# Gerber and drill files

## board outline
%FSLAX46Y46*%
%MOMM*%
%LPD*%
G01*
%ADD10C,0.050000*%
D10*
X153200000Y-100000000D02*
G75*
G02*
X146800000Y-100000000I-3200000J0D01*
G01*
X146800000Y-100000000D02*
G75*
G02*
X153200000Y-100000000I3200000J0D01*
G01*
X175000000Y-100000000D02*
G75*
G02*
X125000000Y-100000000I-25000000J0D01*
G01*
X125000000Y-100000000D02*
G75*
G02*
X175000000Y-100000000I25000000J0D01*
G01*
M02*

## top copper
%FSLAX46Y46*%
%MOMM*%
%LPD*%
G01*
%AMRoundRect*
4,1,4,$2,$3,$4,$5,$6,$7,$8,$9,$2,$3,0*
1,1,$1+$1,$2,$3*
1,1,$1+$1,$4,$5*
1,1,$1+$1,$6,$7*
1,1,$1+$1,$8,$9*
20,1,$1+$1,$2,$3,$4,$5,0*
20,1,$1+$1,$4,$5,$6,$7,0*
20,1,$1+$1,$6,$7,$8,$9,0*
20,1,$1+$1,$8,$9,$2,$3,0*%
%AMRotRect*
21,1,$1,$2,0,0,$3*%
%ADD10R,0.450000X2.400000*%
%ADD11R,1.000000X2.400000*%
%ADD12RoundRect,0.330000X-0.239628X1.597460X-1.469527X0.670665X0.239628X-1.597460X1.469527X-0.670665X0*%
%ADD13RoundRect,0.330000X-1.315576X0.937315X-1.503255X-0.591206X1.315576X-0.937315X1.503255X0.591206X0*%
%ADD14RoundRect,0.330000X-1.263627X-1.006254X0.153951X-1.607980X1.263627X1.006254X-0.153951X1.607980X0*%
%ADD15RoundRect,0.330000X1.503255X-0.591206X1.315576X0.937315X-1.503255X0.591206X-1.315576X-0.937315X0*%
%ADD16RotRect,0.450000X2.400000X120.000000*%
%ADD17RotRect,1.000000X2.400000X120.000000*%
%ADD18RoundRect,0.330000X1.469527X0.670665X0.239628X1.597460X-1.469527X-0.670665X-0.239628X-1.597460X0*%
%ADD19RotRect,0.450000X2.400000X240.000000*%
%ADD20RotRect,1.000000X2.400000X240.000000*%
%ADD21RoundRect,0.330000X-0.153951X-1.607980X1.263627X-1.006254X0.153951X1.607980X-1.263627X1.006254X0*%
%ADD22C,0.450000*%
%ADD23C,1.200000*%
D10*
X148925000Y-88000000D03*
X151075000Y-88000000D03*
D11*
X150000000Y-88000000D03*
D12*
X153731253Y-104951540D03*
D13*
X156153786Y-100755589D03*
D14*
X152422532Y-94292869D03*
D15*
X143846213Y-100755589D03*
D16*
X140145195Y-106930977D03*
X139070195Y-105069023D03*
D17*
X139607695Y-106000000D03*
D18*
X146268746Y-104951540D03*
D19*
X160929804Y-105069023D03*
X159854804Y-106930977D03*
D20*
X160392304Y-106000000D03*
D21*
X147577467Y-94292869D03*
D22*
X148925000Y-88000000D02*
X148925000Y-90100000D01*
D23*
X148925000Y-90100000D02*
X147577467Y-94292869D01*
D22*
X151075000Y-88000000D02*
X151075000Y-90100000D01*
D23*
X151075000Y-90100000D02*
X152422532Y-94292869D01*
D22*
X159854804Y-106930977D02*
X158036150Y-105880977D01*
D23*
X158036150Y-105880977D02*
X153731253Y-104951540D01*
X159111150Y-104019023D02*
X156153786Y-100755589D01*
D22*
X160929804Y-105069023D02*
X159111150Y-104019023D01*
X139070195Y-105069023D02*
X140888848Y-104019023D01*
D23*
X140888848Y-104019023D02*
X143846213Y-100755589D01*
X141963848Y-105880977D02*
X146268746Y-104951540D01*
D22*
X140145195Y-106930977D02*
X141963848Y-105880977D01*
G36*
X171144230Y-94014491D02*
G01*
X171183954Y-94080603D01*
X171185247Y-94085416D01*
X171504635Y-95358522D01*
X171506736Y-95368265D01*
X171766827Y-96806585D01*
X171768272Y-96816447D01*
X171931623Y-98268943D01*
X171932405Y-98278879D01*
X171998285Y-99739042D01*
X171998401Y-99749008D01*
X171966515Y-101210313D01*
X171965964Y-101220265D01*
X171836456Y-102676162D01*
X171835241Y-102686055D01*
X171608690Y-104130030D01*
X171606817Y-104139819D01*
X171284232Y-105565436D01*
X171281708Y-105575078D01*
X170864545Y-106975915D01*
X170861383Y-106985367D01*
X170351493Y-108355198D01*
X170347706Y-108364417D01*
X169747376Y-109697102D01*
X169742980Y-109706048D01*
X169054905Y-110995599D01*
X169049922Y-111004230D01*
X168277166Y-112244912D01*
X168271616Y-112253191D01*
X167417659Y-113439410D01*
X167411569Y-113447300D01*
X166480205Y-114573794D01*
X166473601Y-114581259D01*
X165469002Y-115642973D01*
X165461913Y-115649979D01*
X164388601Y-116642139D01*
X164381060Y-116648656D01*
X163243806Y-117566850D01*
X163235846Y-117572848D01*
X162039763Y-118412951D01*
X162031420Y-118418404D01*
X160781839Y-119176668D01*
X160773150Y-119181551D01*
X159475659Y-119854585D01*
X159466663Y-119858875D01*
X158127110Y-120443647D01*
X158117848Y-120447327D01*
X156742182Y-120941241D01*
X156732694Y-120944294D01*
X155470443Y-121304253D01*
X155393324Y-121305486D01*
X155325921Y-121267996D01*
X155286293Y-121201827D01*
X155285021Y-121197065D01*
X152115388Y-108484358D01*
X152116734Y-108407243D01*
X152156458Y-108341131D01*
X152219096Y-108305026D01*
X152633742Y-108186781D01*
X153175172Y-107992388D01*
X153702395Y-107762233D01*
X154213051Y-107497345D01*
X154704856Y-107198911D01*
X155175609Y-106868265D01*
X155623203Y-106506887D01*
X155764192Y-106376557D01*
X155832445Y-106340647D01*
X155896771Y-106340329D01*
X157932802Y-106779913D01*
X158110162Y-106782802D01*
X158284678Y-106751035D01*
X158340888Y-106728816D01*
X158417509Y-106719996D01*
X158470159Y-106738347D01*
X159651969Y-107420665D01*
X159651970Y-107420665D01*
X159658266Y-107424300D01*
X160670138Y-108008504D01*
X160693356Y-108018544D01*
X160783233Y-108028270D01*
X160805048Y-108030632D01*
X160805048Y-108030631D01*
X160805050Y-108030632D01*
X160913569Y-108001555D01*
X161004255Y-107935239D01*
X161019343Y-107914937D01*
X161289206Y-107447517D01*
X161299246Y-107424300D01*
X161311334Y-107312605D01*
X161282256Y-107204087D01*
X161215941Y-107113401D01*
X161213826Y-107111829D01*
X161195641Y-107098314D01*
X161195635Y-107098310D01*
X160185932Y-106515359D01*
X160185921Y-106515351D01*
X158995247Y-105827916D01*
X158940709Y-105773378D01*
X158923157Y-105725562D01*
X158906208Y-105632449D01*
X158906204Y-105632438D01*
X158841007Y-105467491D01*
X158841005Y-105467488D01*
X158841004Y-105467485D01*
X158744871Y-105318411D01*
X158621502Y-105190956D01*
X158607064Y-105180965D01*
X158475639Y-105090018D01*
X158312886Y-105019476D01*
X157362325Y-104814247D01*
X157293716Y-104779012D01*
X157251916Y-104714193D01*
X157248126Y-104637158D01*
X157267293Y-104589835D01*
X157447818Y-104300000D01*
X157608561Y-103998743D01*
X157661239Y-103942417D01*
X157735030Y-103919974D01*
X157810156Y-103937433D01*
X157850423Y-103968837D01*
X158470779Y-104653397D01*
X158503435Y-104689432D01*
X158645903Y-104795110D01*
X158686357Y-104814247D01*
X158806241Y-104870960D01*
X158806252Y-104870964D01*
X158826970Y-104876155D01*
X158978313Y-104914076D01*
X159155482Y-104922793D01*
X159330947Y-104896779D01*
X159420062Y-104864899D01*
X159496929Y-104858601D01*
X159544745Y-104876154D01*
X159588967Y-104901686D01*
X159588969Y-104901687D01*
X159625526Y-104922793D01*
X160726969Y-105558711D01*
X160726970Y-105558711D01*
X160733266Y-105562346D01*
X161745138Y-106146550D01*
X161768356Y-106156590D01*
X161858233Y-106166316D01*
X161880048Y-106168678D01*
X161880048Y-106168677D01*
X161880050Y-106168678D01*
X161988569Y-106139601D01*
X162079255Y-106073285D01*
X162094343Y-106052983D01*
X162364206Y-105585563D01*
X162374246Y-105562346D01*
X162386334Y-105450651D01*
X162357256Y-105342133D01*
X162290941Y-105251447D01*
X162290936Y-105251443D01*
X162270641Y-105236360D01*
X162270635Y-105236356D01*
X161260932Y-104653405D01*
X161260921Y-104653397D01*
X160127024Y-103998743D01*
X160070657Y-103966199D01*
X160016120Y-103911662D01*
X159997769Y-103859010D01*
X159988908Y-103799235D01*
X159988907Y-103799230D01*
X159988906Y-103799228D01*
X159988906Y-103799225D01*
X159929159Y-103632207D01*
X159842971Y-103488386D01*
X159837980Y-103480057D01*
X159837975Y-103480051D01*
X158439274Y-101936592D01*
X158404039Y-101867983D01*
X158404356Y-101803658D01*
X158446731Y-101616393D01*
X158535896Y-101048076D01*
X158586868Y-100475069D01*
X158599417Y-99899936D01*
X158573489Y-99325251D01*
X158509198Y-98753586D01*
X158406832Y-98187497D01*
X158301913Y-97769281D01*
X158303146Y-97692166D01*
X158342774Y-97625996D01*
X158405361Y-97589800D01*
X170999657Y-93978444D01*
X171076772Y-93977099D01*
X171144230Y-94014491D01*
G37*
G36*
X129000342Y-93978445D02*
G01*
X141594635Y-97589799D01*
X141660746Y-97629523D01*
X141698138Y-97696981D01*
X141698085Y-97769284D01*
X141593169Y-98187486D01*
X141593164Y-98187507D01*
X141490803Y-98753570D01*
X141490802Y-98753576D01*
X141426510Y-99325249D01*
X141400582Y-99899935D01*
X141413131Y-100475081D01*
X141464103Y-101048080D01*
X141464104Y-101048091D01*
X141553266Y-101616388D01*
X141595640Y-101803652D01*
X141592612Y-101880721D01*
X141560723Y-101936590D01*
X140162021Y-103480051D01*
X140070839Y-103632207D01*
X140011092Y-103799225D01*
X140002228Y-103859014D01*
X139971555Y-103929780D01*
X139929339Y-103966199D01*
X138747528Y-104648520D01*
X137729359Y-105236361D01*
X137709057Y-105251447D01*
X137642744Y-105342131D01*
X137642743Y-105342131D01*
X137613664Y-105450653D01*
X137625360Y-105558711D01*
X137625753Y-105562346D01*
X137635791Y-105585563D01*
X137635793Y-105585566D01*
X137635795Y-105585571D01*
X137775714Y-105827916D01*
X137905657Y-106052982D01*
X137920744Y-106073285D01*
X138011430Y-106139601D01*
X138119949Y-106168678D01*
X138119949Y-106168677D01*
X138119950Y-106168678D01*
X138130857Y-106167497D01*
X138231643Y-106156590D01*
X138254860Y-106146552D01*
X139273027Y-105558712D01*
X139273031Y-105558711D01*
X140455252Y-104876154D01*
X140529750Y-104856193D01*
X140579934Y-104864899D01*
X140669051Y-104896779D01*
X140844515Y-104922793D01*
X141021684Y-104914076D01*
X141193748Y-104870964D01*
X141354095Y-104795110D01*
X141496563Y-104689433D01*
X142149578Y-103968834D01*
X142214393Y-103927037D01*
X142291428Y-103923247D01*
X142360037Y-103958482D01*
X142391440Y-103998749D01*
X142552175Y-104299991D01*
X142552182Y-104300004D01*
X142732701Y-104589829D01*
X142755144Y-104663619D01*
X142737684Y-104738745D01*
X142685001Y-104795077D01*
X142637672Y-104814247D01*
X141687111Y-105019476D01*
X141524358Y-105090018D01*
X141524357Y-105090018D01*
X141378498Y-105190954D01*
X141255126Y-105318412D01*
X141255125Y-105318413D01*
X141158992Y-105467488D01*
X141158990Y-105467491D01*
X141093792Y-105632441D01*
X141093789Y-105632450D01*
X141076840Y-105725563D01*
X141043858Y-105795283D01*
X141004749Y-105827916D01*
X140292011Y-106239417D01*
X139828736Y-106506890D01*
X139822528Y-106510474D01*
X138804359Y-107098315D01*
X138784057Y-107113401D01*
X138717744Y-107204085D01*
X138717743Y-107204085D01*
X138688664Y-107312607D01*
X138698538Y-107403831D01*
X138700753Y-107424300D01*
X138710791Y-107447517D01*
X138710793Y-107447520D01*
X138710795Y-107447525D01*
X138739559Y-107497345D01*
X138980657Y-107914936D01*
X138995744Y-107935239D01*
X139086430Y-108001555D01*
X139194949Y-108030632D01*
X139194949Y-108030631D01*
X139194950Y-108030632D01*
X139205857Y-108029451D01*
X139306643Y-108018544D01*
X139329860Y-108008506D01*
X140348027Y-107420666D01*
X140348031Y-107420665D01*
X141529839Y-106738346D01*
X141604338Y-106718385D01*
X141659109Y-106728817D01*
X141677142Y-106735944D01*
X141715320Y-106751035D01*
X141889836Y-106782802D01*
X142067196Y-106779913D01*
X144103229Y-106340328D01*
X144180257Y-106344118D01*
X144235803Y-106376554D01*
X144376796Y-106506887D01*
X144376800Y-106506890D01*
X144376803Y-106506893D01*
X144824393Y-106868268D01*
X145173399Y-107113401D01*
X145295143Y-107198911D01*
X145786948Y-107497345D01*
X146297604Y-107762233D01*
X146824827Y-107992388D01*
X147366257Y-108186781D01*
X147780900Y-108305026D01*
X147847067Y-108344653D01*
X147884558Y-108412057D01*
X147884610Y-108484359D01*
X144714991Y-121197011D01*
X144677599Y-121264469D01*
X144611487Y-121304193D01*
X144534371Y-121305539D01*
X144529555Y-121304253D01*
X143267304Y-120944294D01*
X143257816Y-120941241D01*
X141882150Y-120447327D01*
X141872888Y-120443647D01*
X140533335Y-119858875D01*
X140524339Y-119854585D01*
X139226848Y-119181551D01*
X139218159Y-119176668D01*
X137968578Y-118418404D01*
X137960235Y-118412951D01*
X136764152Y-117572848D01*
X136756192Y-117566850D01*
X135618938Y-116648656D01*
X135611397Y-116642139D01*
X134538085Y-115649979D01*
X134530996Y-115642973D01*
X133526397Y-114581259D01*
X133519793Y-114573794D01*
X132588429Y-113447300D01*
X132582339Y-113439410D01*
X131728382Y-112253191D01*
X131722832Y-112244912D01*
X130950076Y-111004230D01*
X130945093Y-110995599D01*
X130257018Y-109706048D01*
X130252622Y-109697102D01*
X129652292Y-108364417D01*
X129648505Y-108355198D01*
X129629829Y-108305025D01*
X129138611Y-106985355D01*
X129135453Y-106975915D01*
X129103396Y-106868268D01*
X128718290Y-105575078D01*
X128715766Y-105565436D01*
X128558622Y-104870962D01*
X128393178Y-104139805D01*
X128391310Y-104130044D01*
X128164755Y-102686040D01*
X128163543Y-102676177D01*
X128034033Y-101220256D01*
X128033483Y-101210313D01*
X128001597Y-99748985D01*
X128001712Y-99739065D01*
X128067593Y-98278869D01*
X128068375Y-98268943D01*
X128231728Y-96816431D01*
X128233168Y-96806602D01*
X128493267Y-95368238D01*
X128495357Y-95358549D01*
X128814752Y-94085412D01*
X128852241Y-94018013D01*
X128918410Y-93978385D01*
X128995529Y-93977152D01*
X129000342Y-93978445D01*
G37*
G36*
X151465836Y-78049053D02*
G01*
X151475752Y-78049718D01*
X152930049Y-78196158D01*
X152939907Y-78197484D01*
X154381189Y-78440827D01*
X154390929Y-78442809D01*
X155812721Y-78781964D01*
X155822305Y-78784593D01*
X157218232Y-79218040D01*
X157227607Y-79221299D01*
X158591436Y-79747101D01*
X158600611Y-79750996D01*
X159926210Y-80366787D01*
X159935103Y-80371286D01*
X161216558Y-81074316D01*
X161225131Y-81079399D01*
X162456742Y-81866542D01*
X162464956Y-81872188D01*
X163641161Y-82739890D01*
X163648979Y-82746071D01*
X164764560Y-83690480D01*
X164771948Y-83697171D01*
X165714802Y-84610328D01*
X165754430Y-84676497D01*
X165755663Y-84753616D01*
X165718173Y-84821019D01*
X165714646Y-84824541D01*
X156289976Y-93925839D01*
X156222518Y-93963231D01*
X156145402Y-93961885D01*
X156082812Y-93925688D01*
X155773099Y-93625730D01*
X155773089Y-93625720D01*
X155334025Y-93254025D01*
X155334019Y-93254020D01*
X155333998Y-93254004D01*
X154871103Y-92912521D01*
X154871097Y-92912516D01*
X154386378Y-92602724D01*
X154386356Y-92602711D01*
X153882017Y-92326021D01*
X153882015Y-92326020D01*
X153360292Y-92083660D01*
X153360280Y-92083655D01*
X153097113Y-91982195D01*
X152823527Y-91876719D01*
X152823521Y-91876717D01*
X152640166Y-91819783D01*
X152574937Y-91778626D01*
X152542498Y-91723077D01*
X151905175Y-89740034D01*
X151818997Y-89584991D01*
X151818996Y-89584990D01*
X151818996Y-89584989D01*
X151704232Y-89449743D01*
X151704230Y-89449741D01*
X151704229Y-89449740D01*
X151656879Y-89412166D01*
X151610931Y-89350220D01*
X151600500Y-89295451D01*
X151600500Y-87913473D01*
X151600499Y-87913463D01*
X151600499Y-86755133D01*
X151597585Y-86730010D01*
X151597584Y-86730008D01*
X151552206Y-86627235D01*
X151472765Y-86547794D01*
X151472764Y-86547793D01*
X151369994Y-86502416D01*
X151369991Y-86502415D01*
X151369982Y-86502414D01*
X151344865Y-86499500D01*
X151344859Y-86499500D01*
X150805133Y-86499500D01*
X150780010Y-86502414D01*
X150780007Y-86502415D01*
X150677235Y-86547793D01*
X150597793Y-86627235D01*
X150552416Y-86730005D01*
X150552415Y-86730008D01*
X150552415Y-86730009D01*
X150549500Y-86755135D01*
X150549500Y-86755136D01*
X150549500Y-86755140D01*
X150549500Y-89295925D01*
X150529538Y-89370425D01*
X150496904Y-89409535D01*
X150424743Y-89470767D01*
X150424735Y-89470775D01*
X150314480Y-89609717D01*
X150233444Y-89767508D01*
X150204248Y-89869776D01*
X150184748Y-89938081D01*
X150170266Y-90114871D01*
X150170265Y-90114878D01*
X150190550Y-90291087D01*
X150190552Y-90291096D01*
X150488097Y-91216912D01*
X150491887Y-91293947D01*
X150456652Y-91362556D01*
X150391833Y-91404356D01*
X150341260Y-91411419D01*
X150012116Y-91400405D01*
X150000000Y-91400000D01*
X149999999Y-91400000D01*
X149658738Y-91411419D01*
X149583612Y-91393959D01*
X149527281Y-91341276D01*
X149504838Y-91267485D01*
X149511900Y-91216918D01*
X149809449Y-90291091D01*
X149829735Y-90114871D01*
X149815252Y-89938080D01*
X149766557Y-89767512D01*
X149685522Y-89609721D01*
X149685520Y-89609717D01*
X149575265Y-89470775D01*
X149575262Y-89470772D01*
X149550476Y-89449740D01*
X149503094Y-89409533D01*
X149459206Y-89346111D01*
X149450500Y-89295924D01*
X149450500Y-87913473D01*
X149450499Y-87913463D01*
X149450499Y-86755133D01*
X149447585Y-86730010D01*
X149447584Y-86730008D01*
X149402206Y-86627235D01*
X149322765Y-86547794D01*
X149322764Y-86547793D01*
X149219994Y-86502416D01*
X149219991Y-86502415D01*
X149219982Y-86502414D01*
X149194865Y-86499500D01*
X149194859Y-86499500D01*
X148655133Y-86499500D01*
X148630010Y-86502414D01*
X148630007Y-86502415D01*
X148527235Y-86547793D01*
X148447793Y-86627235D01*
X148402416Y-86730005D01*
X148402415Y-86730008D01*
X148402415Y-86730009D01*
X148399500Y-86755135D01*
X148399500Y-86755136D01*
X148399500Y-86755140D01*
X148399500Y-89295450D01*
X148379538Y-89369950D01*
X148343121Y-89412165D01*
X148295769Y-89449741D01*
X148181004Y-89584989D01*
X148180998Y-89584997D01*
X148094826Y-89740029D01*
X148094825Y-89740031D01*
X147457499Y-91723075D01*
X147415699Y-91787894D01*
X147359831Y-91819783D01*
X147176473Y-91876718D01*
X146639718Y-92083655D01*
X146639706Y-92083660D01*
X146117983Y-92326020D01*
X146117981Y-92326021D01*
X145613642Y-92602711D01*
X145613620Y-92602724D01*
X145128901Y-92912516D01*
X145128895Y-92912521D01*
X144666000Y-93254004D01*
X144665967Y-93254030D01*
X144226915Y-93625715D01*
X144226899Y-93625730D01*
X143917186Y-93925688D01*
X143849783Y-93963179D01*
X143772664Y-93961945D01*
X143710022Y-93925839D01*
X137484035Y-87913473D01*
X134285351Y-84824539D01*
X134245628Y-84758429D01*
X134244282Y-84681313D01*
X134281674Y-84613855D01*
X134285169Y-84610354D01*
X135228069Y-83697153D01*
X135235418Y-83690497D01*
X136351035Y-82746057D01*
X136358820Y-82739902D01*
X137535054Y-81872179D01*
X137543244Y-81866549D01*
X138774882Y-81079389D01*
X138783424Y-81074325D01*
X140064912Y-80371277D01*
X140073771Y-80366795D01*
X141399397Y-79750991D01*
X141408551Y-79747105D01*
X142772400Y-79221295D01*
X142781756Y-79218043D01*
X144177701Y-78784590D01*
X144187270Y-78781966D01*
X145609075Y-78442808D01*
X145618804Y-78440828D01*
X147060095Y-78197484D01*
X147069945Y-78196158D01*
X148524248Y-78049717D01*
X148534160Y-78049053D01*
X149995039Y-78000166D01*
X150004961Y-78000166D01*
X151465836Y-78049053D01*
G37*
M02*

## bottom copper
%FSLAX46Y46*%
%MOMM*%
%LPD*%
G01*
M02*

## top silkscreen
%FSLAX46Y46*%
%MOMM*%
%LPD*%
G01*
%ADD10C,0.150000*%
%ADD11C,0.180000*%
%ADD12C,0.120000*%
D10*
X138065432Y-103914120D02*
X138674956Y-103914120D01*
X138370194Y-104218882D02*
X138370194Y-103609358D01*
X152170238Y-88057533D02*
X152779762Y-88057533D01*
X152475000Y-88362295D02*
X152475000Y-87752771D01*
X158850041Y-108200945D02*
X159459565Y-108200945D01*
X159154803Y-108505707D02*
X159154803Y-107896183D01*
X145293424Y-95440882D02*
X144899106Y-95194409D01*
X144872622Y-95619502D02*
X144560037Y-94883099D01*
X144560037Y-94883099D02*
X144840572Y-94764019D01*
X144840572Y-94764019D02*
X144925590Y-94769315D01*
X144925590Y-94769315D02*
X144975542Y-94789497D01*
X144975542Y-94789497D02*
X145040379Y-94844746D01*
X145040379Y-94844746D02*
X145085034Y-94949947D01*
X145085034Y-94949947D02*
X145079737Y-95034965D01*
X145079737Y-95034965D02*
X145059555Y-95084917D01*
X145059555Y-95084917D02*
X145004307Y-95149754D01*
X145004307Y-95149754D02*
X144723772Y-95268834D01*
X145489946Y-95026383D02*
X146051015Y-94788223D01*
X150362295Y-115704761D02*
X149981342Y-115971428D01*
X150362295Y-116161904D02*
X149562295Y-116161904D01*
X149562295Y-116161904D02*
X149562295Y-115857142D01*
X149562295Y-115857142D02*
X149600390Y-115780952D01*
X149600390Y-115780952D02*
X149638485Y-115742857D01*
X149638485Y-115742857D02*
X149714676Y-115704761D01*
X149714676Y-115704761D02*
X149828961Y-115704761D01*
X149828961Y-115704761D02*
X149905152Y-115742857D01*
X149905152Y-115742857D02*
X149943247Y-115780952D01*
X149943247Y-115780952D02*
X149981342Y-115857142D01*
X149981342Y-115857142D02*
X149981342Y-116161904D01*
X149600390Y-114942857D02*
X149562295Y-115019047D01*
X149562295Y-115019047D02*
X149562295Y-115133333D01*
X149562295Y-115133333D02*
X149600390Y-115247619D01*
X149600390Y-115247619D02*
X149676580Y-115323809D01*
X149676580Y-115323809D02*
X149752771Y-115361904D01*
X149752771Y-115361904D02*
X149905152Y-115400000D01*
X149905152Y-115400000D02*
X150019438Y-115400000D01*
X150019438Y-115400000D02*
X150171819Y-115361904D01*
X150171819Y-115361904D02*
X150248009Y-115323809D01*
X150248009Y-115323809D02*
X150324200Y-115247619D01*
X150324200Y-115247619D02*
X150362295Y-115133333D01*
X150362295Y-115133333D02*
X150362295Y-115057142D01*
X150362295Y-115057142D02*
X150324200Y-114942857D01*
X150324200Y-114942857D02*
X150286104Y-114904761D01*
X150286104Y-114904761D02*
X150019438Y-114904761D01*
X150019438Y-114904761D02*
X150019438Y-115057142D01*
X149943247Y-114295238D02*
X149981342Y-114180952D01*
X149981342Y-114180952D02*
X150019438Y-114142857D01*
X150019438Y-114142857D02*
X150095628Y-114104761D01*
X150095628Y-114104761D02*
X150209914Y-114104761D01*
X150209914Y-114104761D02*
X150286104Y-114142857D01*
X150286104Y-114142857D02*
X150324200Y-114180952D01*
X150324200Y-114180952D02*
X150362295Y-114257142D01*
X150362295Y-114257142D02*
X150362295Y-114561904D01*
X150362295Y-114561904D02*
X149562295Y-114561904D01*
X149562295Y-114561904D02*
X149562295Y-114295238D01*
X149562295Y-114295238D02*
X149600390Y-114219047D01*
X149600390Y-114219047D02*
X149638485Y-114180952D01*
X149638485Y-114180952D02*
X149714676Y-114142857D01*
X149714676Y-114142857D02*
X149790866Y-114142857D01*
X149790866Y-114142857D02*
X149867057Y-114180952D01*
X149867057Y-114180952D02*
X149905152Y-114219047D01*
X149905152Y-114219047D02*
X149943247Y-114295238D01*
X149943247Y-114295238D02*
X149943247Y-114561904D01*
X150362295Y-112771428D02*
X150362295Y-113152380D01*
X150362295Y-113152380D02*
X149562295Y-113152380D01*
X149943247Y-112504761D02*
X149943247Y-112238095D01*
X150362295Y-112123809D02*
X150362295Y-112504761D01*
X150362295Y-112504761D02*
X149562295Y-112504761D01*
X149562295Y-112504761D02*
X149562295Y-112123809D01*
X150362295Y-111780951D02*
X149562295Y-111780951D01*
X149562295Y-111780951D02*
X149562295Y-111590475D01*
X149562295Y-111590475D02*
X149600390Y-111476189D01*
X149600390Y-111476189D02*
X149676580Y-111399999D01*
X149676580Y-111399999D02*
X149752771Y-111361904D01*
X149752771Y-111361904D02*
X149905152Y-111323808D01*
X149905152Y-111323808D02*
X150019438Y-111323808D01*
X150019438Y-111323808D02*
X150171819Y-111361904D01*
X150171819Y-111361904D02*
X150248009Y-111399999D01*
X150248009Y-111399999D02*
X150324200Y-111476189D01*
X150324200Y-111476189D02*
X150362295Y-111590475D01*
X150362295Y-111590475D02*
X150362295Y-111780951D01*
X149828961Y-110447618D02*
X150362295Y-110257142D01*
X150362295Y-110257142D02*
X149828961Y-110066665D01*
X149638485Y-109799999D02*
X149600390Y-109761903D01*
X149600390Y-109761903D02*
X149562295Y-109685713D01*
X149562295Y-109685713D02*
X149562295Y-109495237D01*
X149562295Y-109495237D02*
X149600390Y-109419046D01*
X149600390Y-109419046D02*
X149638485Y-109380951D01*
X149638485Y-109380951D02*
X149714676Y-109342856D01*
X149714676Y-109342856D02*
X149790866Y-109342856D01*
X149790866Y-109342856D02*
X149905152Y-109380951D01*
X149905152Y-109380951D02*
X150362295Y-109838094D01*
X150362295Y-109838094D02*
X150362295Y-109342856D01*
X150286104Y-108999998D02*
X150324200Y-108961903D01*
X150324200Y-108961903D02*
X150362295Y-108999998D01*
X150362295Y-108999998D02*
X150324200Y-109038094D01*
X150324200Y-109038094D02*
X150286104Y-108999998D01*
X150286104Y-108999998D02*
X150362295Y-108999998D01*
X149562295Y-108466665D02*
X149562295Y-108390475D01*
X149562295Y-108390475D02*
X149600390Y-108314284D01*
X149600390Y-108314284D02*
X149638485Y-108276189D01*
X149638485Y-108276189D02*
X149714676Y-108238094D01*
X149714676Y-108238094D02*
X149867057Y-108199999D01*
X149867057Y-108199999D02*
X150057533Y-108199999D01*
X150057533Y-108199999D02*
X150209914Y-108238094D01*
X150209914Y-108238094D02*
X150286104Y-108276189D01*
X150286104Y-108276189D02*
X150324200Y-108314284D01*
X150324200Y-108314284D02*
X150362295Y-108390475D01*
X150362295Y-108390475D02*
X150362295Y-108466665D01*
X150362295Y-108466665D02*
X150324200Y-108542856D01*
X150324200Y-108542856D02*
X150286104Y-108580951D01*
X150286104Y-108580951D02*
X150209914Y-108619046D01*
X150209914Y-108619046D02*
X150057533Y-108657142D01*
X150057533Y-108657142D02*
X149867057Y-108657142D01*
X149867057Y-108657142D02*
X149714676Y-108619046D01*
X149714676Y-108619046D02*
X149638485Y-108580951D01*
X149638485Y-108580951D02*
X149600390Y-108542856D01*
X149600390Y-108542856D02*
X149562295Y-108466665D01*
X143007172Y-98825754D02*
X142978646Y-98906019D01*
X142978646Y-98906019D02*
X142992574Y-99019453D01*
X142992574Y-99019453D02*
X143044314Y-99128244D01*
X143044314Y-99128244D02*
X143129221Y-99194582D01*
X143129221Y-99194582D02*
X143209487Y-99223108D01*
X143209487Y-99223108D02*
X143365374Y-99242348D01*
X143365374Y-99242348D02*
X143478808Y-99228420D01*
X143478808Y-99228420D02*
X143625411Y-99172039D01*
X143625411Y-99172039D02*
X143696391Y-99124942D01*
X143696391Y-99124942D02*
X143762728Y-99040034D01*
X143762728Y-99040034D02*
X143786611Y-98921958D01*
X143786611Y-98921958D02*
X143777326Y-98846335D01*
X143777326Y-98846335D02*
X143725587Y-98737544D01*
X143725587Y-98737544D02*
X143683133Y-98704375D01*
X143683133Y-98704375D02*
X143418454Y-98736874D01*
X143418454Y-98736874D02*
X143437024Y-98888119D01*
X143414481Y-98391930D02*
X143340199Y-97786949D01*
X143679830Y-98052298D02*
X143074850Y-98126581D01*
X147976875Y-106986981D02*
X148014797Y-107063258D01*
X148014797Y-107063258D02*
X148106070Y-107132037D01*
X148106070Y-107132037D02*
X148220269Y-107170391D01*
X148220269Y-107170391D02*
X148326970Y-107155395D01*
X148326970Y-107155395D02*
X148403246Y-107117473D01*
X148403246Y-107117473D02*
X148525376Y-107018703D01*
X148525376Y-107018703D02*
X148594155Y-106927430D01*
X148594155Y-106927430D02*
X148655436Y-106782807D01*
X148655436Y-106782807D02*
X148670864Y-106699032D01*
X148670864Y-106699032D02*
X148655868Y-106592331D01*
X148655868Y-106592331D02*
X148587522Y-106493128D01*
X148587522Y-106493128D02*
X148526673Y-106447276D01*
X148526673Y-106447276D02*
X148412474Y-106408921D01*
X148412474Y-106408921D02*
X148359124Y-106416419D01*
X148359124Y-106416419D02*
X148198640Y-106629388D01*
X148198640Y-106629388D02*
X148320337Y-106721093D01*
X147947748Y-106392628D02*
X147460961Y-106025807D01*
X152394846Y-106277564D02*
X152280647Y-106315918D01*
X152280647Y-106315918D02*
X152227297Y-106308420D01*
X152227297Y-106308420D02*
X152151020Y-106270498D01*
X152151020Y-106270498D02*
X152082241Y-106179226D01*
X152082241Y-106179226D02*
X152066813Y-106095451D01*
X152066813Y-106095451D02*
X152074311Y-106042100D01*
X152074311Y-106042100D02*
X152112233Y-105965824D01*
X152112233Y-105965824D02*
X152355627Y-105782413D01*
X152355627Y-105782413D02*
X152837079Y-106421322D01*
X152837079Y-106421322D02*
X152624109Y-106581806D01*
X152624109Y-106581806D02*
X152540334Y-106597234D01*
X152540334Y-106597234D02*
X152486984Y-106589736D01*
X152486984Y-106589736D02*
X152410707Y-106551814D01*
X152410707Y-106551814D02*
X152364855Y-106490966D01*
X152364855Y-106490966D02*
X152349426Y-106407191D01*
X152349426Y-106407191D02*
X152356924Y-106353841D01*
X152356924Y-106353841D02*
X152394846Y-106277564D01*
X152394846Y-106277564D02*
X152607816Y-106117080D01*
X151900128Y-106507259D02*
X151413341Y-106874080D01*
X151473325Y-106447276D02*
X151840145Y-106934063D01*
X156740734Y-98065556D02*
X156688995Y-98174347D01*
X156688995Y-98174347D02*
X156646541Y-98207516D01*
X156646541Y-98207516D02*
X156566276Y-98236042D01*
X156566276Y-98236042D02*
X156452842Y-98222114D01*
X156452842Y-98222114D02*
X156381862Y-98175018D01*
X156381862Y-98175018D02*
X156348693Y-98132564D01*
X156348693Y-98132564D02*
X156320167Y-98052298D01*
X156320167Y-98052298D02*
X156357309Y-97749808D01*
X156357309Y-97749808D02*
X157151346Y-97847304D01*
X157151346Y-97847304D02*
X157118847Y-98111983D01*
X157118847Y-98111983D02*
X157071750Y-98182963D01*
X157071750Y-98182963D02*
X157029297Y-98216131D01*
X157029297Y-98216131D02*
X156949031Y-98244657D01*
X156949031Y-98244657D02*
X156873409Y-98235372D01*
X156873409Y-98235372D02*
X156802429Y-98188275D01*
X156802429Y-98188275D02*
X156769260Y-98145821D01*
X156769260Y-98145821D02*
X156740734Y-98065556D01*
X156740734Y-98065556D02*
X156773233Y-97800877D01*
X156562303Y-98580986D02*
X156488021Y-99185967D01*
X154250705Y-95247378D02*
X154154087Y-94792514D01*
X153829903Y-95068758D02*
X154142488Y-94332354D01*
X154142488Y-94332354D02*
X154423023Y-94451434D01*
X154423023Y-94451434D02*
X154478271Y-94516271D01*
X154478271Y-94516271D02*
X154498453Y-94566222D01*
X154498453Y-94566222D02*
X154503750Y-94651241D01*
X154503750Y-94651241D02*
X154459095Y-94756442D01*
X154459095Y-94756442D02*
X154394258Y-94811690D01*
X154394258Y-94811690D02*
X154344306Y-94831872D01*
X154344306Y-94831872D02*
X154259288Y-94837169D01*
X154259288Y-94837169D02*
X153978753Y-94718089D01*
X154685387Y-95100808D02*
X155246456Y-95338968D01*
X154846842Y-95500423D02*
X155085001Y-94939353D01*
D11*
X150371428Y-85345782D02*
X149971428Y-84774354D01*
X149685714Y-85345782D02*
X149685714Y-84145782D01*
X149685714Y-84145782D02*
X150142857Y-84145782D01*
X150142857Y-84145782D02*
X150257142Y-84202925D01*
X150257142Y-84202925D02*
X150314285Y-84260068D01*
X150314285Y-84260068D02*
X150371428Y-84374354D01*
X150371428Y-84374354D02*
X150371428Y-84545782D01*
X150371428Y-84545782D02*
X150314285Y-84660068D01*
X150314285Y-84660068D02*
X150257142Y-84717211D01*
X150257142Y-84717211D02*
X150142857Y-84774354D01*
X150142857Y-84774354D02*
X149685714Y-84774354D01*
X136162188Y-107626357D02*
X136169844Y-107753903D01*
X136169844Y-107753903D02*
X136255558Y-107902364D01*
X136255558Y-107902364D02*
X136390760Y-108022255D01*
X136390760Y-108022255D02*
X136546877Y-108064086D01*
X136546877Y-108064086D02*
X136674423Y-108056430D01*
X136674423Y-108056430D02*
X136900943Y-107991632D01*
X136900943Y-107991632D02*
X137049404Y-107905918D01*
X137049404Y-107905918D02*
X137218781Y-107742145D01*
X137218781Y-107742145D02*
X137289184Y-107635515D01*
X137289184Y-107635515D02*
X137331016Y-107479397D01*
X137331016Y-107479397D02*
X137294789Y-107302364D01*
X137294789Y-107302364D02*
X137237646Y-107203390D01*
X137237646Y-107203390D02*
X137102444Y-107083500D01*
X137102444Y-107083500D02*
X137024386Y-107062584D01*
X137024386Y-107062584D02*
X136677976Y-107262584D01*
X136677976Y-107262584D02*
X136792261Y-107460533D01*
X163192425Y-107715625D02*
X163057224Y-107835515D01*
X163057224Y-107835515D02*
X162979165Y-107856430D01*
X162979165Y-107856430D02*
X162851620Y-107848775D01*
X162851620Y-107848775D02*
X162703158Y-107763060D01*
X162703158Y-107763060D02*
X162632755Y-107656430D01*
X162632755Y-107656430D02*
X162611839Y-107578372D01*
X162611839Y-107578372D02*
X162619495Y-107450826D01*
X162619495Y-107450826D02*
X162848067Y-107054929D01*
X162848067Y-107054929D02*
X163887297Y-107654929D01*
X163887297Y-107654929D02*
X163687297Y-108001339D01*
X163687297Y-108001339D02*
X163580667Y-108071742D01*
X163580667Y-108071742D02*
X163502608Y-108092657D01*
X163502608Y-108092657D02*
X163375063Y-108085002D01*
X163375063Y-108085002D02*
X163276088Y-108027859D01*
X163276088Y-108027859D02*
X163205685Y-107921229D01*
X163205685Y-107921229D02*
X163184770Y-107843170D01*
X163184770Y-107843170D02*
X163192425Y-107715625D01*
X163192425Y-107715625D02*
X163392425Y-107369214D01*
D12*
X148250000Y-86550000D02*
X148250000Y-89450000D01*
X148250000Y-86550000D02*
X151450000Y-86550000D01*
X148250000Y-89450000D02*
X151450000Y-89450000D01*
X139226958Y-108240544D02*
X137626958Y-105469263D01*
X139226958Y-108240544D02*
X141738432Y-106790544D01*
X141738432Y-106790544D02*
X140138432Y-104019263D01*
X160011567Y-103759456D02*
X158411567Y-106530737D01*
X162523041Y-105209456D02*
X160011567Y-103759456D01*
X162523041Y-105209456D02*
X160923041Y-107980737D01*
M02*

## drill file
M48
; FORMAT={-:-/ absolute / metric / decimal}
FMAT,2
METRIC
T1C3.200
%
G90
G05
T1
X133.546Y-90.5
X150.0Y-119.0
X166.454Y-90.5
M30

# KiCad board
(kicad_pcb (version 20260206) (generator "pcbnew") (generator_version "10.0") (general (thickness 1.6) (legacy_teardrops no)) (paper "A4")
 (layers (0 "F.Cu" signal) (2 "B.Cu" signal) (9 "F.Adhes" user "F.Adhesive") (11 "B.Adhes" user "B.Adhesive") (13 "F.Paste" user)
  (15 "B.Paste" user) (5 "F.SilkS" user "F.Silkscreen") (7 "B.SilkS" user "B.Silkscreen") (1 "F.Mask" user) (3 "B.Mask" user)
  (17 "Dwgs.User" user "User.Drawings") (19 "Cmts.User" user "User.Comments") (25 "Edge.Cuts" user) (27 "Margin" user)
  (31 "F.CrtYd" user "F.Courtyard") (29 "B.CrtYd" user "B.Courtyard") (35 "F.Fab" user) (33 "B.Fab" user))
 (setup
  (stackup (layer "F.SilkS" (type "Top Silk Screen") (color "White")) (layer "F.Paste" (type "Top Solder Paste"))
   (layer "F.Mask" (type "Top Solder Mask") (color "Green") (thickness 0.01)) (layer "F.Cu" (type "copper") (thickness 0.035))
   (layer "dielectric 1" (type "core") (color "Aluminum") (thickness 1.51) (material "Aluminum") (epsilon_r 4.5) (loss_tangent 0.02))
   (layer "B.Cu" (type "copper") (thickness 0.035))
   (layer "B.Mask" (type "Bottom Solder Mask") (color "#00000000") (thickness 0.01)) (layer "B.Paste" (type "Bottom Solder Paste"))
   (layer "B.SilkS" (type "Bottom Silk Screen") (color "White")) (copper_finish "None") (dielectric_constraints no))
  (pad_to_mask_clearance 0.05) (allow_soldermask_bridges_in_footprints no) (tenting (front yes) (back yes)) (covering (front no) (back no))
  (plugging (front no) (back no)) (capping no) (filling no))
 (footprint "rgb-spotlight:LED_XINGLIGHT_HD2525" (layer "F.Cu") (at 150 88)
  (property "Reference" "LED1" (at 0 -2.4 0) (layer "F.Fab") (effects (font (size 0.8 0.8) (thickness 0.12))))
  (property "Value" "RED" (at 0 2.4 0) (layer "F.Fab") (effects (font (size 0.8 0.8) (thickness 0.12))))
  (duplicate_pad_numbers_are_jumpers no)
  (fp_line (start -1.75 -1.45) (end -1.75 1.45) (stroke (width 0.12) (type solid)) (layer "F.SilkS"))
  (fp_line (start -1.75 -1.45) (end 1.45 -1.45) (stroke (width 0.12) (type solid)) (layer "F.SilkS"))
  (fp_line (start -1.75 1.45) (end 1.45 1.45) (stroke (width 0.12) (type solid)) (layer "F.SilkS"))
  (pad "1" smd rect (at -1.075 0) (size 0.45 2.4) (layers "F.Cu" "F.Mask" "F.Paste") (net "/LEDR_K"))
  (pad "2" smd rect (at 1.075 0) (size 0.45 2.4) (layers "F.Cu" "F.Mask" "F.Paste") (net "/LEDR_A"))
  (pad "3" smd rect (at 0 0) (size 1 2.4) (layers "F.Cu" "F.Mask" "F.Paste") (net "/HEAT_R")))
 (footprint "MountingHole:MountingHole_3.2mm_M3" (layer "F.Cu") (at 133.545517 90.5)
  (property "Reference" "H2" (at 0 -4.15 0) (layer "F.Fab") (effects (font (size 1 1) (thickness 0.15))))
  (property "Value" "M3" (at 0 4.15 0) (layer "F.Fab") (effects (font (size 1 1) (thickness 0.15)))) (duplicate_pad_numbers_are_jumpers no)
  (pad "" np_thru_hole circle (at 0 0) (size 3.2 3.2) (drill 3.2) (layers "*.Cu" "*.Mask")))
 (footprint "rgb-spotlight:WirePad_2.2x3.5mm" (layer "F.Cu") (at 153.731253 104.95154 -143)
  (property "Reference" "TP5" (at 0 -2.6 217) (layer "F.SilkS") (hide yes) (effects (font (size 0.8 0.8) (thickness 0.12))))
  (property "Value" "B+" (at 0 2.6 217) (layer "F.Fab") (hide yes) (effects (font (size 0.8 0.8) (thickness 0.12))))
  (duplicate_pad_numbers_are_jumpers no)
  (pad "1" smd roundrect (at 0 0 217) (size 2.2 3.5) (layers "F.Cu" "F.Mask") (roundrect_rratio 0.15) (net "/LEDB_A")))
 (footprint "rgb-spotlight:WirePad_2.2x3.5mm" (layer "F.Cu") (at 156.153786 100.755589 -97)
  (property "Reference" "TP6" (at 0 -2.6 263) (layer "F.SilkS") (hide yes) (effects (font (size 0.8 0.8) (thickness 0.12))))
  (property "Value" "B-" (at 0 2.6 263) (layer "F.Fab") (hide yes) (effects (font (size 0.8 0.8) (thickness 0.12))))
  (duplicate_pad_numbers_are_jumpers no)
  (pad "1" smd roundrect (at 0 0 263) (size 2.2 3.5) (layers "F.Cu" "F.Mask") (roundrect_rratio 0.15) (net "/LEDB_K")))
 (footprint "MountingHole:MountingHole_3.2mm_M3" (layer "F.Cu") (at 166.454482 90.5)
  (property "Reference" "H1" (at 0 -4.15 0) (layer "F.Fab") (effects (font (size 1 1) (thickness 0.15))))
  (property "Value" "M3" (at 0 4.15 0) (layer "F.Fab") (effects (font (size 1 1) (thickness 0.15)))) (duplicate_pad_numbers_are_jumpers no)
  (pad "" np_thru_hole circle (at 0 0) (size 3.2 3.2) (drill 3.2) (layers "*.Cu" "*.Mask")))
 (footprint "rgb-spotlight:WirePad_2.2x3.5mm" (layer "F.Cu") (at 152.422532 94.292869 -23)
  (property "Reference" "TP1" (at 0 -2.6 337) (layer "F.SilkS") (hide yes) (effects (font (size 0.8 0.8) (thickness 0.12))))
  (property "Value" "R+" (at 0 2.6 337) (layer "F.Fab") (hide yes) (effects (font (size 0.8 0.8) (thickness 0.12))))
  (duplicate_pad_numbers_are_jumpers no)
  (pad "1" smd roundrect (at 0 0 337) (size 2.2 3.5) (layers "F.Cu" "F.Mask") (roundrect_rratio 0.15) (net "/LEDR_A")))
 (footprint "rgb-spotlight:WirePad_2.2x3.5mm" (layer "F.Cu") (at 143.846213 100.755589 97)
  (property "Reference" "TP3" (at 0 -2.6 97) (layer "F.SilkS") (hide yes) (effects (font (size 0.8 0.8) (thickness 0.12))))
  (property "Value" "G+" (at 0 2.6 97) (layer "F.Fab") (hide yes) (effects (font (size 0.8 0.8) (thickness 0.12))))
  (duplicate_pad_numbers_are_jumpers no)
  (pad "1" smd roundrect (at 0 0 97) (size 2.2 3.5) (layers "F.Cu" "F.Mask") (roundrect_rratio 0.15) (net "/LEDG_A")))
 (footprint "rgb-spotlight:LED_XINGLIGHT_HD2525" (layer "F.Cu") (at 139.607695 106 120)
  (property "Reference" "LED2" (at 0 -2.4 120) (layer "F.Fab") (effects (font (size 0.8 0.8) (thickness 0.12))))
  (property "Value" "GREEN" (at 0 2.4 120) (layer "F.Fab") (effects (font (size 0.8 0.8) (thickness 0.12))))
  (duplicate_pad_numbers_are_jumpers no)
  (fp_line (start -1.75 -1.45) (end 1.45 -1.45) (stroke (width 0.12) (type solid)) (layer "F.SilkS"))
  (fp_line (start -1.75 -1.45) (end -1.75 1.45) (stroke (width 0.12) (type solid)) (layer "F.SilkS"))
  (fp_line (start -1.75 1.45) (end 1.45 1.45) (stroke (width 0.12) (type solid)) (layer "F.SilkS"))
  (pad "1" smd rect (at -1.075 0 120) (size 0.45 2.4) (layers "F.Cu" "F.Mask" "F.Paste") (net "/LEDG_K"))
  (pad "2" smd rect (at 1.075 0 120) (size 0.45 2.4) (layers "F.Cu" "F.Mask" "F.Paste") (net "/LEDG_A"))
  (pad "3" smd rect (at 0 0 120) (size 1 2.4) (layers "F.Cu" "F.Mask" "F.Paste") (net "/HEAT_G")))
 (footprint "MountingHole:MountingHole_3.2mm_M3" (layer "F.Cu") (at 150 119)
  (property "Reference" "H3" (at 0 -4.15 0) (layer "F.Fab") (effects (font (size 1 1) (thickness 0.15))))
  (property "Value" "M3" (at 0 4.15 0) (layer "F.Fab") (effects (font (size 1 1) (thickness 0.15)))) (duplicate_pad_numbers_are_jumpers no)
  (pad "" np_thru_hole circle (at 0 0) (size 3.2 3.2) (drill 3.2) (layers "*.Cu" "*.Mask")))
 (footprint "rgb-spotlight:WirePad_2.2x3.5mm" (layer "F.Cu") (at 146.268746 104.95154 143)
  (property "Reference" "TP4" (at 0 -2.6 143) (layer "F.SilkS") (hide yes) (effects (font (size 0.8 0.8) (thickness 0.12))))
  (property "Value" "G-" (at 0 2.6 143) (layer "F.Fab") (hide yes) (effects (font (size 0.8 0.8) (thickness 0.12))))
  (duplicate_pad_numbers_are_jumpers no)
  (pad "1" smd roundrect (at 0 0 143) (size 2.2 3.5) (layers "F.Cu" "F.Mask") (roundrect_rratio 0.15) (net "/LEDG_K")))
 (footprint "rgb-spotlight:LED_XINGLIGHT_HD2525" (layer "F.Cu") (at 160.392304 106 -120)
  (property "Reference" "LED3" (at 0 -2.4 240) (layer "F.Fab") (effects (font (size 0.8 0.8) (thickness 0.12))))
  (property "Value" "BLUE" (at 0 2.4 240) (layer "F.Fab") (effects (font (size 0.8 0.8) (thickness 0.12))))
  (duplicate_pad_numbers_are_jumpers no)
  (fp_line (start -1.75 1.45) (end 1.45 1.45) (stroke (width 0.12) (type solid)) (layer "F.SilkS"))
  (fp_line (start -1.75 -1.45) (end -1.75 1.45) (stroke (width 0.12) (type solid)) (layer "F.SilkS"))
  (fp_line (start -1.75 -1.45) (end 1.45 -1.45) (stroke (width 0.12) (type solid)) (layer "F.SilkS"))
  (pad "1" smd rect (at -1.075 0 240) (size 0.45 2.4) (layers "F.Cu" "F.Mask" "F.Paste") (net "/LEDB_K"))
  (pad "2" smd rect (at 1.075 0 240) (size 0.45 2.4) (layers "F.Cu" "F.Mask" "F.Paste") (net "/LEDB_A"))
  (pad "3" smd rect (at 0 0 240) (size 1 2.4) (layers "F.Cu" "F.Mask" "F.Paste") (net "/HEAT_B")))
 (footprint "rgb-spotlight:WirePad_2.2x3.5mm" (layer "F.Cu") (at 147.577467 94.292869 23)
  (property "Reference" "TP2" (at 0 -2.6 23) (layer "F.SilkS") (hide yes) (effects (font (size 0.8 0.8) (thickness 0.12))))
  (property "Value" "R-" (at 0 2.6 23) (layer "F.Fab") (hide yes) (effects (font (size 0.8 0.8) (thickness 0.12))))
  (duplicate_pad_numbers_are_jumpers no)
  (pad "1" smd roundrect (at 0 0 23) (size 2.2 3.5) (layers "F.Cu" "F.Mask") (roundrect_rratio 0.15) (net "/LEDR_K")))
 (gr_circle (center 150 100) (end 153.2 100) (stroke (width 0.05) (type default)) (fill no) (layer "Edge.Cuts"))
 (gr_circle (center 150 100) (end 175 100) (stroke (width 0.05) (type default)) (fill no) (layer "Edge.Cuts"))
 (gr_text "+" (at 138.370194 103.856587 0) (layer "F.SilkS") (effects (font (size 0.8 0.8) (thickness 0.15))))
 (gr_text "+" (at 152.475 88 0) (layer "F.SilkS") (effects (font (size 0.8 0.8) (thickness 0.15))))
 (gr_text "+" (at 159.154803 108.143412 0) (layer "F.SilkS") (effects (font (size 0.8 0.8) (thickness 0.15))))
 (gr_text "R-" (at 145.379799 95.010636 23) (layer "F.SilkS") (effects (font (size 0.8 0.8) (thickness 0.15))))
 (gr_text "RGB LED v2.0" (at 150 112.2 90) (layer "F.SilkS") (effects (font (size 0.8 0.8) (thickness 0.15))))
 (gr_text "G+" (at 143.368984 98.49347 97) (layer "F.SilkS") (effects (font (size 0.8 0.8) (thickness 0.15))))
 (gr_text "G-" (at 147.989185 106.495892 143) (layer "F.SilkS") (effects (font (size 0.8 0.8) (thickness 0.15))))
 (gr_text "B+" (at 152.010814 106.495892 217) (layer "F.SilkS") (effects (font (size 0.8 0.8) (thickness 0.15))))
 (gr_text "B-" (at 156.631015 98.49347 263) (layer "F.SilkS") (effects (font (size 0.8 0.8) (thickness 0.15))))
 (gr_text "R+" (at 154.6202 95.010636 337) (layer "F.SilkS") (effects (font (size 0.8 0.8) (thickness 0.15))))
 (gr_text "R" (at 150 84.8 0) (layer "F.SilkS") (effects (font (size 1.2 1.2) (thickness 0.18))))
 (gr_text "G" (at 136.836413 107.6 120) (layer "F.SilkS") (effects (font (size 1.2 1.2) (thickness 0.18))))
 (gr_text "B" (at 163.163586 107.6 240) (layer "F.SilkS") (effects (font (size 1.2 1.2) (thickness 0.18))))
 (segment (start 148.925 88) (end 148.925 90.1) (width 0.45) (layer "F.Cu") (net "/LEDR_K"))
 (segment (start 148.925 90.1) (end 147.577467 94.292869) (width 1.2) (layer "F.Cu") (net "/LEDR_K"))
 (segment (start 151.075 88) (end 151.075 90.1) (width 0.45) (layer "F.Cu") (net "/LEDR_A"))
 (segment (start 151.075 90.1) (end 152.422532 94.292869) (width 1.2) (layer "F.Cu") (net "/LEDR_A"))
 (segment (start 159.854804 106.930977) (end 158.03615 105.880977) (width 0.45) (layer "F.Cu") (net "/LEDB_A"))
 (segment (start 158.03615 105.880977) (end 153.731253 104.95154) (width 1.2) (layer "F.Cu") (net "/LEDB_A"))
 (segment (start 159.11115 104.019023) (end 156.153786 100.755589) (width 1.2) (layer "F.Cu") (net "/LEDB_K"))
 (segment (start 160.929804 105.069023) (end 159.11115 104.019023) (width 0.45) (layer "F.Cu") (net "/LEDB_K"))
 (segment (start 139.070195 105.069023) (end 140.888848 104.019023) (width 0.45) (layer "F.Cu") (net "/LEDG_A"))
 (segment (start 140.888848 104.019023) (end 143.846213 100.755589) (width 1.2) (layer "F.Cu") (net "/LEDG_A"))
 (segment (start 141.963848 105.880977) (end 146.268746 104.95154) (width 1.2) (layer "F.Cu") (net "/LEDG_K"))
 (segment (start 140.145195 106.930977) (end 141.963848 105.880977) (width 0.45) (layer "F.Cu") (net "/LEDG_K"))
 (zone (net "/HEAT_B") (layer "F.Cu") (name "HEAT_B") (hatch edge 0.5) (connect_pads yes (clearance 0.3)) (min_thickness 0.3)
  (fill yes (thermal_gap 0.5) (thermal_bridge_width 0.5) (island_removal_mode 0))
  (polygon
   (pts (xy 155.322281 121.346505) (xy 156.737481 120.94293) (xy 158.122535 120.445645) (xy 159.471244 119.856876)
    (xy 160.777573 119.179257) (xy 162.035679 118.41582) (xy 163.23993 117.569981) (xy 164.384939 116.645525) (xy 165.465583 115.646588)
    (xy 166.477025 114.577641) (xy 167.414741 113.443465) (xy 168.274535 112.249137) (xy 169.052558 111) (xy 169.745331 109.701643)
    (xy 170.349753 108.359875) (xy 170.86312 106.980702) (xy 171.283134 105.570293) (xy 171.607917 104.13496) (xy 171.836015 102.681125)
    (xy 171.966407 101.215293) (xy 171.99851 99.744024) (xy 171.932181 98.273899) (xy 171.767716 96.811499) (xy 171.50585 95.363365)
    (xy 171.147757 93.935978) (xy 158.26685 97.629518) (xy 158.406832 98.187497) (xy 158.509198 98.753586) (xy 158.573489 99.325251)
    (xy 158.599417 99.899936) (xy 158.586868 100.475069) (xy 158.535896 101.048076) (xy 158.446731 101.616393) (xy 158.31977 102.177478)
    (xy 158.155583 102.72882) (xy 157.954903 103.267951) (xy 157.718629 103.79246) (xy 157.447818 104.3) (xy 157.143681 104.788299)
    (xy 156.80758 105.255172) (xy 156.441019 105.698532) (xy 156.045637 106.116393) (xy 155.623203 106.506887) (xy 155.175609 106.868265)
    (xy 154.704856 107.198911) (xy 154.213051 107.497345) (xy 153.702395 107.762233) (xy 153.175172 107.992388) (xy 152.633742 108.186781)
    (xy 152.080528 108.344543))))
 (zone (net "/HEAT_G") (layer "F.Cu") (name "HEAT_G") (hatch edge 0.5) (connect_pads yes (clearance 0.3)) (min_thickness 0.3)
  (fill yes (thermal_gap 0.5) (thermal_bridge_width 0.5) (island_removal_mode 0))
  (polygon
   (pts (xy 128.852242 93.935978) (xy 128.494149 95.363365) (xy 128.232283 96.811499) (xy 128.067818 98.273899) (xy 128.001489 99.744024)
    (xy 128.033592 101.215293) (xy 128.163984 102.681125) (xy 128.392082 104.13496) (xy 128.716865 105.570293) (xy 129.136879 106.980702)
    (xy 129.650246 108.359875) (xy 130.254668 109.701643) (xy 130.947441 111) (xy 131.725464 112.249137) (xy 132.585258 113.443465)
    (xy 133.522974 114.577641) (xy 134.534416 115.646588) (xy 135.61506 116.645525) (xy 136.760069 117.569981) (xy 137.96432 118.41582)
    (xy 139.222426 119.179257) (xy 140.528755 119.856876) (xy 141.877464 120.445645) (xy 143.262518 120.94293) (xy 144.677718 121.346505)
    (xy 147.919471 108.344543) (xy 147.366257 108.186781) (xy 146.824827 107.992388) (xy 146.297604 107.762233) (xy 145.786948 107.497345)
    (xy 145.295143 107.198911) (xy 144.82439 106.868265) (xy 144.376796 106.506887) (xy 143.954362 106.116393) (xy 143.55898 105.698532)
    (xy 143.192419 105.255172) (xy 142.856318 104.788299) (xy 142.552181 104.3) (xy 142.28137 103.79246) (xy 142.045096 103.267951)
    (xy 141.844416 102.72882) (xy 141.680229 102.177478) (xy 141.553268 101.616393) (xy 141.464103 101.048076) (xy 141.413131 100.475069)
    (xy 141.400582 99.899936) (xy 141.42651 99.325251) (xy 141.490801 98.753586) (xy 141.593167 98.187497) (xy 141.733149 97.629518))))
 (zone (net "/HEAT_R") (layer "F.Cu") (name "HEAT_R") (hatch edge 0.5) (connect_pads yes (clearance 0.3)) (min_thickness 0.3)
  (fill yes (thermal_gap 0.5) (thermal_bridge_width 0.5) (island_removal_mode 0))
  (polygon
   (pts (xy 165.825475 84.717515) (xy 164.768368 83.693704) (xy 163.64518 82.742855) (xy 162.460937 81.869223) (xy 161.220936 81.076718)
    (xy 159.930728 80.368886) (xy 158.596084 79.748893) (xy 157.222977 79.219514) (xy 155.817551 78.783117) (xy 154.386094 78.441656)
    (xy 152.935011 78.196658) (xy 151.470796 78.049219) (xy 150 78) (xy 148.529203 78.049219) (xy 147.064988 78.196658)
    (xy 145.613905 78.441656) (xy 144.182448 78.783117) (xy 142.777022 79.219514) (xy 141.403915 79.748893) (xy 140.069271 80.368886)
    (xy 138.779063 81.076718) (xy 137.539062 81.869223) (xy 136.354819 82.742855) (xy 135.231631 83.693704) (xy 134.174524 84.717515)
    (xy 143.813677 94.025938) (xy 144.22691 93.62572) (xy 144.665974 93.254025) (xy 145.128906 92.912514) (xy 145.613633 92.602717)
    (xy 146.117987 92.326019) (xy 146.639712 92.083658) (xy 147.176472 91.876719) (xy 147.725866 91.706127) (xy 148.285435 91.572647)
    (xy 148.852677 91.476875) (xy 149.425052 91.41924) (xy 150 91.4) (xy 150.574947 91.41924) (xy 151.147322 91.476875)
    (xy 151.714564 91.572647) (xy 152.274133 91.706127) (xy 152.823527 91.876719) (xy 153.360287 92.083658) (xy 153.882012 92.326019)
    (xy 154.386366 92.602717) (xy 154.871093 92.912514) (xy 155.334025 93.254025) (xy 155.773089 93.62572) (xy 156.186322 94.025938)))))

